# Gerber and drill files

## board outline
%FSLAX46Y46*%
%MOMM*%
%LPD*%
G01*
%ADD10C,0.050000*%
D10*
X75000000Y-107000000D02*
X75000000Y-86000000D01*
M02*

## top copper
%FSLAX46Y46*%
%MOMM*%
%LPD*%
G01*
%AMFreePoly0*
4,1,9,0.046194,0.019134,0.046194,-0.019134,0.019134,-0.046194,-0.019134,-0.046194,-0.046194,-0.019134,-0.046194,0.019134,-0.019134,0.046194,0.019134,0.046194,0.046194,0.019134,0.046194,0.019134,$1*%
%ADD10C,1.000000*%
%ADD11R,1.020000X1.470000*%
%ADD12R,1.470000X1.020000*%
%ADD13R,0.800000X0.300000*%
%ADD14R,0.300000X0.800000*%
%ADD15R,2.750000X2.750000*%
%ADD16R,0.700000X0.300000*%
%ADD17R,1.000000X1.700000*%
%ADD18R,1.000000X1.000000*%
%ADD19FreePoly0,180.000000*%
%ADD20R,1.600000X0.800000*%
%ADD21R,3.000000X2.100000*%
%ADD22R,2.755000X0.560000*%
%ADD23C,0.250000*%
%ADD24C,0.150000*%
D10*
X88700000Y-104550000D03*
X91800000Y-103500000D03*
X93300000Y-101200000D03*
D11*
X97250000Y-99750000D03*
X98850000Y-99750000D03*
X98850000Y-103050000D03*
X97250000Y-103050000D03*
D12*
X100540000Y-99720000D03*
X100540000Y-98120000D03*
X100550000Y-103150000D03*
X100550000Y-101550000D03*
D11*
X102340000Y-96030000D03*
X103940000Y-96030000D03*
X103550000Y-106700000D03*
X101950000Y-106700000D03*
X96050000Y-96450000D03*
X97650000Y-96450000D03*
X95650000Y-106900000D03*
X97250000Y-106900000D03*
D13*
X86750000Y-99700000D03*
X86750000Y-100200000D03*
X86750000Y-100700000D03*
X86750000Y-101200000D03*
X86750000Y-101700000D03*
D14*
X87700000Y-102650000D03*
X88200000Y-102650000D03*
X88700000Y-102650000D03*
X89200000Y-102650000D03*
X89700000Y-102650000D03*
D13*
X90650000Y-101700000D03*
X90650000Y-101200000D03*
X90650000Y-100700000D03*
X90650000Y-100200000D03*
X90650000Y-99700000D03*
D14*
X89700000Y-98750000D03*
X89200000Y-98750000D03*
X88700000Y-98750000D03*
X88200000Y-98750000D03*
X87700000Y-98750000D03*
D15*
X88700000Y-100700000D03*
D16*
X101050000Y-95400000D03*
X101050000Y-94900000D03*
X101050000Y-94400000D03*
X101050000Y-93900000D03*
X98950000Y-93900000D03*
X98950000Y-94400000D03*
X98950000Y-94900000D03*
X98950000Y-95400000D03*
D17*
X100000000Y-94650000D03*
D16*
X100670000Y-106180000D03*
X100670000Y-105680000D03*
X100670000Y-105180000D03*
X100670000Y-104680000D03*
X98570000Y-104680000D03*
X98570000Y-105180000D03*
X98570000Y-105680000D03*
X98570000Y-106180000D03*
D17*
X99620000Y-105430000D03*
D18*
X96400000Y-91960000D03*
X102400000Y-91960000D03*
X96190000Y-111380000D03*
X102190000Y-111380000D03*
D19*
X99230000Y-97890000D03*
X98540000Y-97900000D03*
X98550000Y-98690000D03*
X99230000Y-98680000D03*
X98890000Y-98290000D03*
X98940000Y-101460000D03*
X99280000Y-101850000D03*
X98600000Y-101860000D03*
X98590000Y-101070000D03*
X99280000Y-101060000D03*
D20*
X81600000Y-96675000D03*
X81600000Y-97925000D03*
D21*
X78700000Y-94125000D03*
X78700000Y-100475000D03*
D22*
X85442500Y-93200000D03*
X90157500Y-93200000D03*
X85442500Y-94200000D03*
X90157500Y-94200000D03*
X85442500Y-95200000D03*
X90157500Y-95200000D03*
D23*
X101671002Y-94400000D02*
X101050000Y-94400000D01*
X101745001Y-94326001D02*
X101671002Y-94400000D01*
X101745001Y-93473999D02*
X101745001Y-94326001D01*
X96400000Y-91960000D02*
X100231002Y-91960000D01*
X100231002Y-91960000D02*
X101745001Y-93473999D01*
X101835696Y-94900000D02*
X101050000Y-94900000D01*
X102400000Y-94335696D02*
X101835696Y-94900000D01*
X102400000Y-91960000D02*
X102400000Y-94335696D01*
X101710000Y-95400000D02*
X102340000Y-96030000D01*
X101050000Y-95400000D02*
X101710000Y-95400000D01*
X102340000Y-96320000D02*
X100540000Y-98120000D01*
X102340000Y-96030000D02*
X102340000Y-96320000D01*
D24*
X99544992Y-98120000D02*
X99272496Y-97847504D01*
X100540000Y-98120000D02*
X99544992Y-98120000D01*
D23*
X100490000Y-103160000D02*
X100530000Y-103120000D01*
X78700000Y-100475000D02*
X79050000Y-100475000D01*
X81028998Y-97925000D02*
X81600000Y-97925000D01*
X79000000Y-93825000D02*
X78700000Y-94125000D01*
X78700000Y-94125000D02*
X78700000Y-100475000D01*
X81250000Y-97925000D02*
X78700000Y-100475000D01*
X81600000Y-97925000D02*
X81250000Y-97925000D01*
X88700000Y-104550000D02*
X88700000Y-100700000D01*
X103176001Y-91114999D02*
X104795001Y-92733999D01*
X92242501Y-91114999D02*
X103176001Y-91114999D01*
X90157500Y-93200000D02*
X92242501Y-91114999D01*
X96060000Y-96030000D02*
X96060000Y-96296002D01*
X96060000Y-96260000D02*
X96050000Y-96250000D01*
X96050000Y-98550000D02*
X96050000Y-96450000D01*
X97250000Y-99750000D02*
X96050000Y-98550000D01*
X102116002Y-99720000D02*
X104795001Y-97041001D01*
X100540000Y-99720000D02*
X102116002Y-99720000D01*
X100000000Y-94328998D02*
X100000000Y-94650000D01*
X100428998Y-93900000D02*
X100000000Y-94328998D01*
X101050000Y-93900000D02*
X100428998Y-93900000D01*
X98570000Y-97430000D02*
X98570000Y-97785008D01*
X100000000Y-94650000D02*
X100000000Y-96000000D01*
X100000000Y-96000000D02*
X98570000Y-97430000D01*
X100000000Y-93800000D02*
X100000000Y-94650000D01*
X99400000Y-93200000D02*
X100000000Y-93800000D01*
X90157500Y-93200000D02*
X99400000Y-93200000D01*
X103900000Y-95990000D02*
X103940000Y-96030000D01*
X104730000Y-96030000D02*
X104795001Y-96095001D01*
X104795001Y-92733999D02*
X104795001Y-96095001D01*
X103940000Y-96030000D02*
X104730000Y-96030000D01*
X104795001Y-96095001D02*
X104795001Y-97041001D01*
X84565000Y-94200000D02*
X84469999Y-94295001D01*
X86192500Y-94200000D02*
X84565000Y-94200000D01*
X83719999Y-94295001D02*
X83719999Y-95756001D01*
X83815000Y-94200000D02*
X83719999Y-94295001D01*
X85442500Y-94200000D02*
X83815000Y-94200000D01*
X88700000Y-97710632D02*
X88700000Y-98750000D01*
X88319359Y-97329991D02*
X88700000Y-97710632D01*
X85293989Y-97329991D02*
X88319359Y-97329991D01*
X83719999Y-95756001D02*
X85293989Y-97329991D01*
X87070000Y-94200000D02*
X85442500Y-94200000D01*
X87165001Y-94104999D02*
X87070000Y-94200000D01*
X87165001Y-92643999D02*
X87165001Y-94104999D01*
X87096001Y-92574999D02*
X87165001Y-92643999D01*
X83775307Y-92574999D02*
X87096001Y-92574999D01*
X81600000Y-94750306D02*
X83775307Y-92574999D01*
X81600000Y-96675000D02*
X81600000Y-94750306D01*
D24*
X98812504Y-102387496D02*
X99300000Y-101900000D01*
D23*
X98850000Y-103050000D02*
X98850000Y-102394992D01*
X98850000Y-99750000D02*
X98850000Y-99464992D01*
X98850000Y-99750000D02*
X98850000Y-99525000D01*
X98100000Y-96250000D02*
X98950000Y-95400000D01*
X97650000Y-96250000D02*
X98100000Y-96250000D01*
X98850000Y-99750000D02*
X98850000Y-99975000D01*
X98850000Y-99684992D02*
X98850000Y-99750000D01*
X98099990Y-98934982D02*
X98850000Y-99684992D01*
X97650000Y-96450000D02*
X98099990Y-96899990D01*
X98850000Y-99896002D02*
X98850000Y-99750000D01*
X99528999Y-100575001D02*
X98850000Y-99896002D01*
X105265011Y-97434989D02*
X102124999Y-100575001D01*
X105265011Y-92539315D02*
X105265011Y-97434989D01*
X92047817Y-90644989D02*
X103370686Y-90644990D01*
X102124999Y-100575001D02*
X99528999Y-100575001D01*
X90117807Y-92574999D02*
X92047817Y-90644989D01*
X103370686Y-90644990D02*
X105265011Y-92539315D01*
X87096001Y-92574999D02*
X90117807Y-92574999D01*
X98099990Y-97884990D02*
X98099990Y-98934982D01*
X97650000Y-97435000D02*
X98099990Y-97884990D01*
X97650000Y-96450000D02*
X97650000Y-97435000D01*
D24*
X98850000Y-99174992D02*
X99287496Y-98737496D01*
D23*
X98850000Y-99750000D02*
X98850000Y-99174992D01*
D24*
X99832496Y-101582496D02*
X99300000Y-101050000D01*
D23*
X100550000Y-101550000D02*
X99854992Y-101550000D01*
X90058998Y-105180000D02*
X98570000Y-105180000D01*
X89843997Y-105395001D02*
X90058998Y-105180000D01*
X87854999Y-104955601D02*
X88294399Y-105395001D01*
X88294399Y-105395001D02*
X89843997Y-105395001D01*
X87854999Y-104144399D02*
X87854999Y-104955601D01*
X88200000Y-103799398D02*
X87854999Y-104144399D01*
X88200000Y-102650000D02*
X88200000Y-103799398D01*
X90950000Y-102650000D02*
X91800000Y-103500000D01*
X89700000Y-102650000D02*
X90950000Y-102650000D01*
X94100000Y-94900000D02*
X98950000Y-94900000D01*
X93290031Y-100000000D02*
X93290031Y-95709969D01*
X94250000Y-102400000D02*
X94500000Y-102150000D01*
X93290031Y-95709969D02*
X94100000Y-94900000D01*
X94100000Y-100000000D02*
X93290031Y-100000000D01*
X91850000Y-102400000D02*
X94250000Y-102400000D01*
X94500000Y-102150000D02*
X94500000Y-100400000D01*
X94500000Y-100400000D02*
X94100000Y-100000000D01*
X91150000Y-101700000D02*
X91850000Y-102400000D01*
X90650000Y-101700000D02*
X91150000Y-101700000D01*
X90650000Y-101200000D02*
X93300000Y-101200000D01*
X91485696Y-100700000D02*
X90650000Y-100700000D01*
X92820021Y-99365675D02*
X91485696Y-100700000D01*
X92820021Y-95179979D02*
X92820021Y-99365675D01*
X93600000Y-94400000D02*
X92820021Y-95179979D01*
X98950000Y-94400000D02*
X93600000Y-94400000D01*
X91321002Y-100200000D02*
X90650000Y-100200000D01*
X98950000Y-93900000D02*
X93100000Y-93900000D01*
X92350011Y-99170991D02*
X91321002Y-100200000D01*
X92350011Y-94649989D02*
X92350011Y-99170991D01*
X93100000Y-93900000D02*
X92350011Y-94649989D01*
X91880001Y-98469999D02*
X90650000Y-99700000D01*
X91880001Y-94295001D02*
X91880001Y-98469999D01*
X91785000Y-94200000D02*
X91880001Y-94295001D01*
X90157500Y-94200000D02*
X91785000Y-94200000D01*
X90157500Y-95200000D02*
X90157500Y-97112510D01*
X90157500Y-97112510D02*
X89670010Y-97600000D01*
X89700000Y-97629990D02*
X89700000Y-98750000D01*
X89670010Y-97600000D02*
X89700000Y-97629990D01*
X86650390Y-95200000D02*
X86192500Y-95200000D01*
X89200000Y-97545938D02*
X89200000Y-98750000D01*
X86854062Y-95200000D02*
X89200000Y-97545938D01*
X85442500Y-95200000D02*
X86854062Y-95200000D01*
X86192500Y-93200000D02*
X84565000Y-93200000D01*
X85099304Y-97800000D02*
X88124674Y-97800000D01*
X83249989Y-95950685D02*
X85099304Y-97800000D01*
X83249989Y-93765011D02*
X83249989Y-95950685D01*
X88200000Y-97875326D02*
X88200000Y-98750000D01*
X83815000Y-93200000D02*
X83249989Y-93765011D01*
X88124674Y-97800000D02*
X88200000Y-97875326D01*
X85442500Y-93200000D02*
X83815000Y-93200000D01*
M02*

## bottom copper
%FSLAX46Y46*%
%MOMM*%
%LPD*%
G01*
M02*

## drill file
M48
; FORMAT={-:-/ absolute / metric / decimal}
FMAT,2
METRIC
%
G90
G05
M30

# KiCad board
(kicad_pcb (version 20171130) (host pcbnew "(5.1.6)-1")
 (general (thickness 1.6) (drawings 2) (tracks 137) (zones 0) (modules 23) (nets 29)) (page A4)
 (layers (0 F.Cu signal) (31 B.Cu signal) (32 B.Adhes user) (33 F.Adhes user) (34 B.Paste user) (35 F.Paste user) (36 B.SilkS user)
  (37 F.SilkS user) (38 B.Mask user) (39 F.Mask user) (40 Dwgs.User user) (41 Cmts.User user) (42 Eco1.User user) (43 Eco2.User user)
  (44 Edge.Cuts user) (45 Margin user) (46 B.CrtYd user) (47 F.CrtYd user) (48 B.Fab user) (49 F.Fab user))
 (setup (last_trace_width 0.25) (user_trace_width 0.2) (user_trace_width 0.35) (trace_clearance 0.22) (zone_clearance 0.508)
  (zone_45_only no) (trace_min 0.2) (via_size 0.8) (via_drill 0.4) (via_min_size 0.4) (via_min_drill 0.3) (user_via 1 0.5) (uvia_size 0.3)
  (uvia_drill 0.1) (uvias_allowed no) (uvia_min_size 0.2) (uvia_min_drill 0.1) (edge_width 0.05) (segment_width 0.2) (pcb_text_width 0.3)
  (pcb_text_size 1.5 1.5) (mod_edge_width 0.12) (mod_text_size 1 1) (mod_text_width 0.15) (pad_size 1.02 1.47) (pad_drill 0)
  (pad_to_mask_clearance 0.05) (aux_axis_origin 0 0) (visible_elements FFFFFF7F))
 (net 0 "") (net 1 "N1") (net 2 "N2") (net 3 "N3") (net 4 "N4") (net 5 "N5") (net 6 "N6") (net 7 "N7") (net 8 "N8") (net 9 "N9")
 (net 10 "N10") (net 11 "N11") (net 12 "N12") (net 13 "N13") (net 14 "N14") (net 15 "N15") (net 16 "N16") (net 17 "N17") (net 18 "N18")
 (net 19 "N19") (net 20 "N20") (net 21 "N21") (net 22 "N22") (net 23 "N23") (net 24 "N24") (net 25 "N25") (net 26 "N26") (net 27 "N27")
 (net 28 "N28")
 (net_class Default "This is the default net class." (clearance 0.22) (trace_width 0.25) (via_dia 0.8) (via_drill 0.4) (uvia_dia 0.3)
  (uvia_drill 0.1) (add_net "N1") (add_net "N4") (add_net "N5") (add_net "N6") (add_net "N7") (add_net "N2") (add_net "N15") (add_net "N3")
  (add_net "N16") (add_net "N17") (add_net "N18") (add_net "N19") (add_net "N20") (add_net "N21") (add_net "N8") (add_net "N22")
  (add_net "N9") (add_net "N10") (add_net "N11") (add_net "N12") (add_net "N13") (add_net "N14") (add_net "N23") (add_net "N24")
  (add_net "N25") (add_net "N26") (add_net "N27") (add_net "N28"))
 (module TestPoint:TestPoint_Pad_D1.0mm (layer F.Cu) (at 88.7 104.55)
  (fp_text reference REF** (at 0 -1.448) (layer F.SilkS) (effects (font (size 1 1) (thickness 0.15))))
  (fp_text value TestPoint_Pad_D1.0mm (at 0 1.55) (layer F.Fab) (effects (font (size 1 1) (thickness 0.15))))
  (pad 1 smd circle (at 0 0) (size 1 1) (layers F.Cu F.Mask) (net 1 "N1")))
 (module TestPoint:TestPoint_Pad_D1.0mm (layer F.Cu) (at 91.8 103.5)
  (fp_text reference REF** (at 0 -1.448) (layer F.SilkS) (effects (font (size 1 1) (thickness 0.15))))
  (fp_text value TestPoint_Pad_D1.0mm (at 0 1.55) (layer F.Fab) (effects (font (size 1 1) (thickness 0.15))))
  (pad 1 smd circle (at 0 0) (size 1 1) (layers F.Cu F.Mask) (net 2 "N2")))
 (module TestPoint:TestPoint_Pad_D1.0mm (layer F.Cu) (at 93.3 101.2)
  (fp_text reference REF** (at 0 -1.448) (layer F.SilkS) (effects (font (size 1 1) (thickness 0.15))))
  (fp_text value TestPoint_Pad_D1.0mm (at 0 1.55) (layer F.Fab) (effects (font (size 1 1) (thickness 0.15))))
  (pad 1 smd circle (at 0 0) (size 1 1) (layers F.Cu F.Mask) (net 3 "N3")))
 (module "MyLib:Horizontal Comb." (layer F.Cu) (at 119.7 96.4)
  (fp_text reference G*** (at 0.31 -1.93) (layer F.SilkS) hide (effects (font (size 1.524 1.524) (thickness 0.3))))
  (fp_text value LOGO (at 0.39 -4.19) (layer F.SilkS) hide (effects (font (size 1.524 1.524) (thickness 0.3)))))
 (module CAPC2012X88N (layer F.Cu) (at 98.05 99.75)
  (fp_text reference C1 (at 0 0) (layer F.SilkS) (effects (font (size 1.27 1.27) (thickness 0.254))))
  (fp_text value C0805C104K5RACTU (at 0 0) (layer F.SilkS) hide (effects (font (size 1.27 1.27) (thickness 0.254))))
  (pad 1 smd rect (at -0.8 0) (size 1.02 1.47) (layers F.Cu F.Paste F.Mask) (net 1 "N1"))
  (pad 2 smd rect (at 0.8 0) (size 1.02 1.47) (layers F.Cu F.Paste F.Mask) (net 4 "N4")))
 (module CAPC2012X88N (layer F.Cu) (at 98.05 103.05)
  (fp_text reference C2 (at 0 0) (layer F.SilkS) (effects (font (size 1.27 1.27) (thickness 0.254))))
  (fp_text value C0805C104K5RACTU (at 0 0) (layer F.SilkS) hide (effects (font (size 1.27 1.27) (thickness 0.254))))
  (pad 2 smd rect (at 0.8 0) (size 1.02 1.47) (layers F.Cu F.Paste F.Mask) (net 4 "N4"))
  (pad 1 smd rect (at -0.8 0) (size 1.02 1.47) (layers F.Cu F.Paste F.Mask) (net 1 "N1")))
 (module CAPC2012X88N (layer F.Cu) (at 100.54 98.92 90)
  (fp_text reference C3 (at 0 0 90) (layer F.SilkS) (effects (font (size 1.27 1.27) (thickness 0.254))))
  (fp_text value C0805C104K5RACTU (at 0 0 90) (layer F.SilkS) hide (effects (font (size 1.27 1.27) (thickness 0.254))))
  (pad 1 smd rect (at -0.8 0 90) (size 1.02 1.47) (layers F.Cu F.Paste F.Mask) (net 1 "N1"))
  (pad 2 smd rect (at 0.8 0 90) (size 1.02 1.47) (layers F.Cu F.Paste F.Mask) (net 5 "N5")))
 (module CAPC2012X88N (layer F.Cu) (at 100.55 102.35 90)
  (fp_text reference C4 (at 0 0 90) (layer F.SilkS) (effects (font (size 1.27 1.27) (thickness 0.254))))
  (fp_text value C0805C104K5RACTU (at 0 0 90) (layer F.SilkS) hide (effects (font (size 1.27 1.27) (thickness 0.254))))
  (pad 1 smd rect (at -0.8 0 90) (size 1.02 1.47) (layers F.Cu F.Paste F.Mask) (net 1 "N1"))
  (pad 2 smd rect (at 0.8 0 90) (size 1.02 1.47) (layers F.Cu F.Paste F.Mask) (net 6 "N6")))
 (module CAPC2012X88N (layer F.Cu) (at 103.14 96.03 180)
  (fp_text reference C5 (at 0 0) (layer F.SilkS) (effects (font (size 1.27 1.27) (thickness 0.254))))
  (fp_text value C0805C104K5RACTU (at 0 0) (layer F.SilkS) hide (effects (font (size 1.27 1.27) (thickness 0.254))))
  (pad 2 smd rect (at 0.8 0 180) (size 1.02 1.47) (layers F.Cu F.Paste F.Mask) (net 5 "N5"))
  (pad 1 smd rect (at -0.8 0 180) (size 1.02 1.47) (layers F.Cu F.Paste F.Mask) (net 1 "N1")))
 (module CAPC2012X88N (layer F.Cu) (at 102.75 106.7 180)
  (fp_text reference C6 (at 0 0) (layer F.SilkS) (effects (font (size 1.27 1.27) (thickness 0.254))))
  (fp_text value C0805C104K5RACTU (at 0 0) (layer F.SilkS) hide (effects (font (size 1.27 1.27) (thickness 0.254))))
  (pad 1 smd rect (at -0.8 0 180) (size 1.02 1.47) (layers F.Cu F.Paste F.Mask) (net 1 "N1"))
  (pad 2 smd rect (at 0.8 0 180) (size 1.02 1.47) (layers F.Cu F.Paste F.Mask) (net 6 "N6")))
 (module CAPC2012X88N (layer F.Cu) (at 96.85 96.45)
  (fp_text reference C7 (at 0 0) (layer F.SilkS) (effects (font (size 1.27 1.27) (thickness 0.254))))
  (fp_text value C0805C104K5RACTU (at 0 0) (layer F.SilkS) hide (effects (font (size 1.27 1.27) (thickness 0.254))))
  (pad 1 smd rect (at -0.8 0) (size 1.02 1.47) (layers F.Cu F.Paste F.Mask) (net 1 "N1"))
  (pad 2 smd rect (at 0.8 0) (size 1.02 1.47) (layers F.Cu F.Paste F.Mask) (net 4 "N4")))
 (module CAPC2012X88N (layer F.Cu) (at 96.45 106.9)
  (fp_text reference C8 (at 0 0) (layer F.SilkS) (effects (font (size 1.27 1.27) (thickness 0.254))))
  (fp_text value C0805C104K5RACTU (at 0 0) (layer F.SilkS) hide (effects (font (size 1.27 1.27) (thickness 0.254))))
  (pad 1 smd rect (at -0.8 0) (size 1.02 1.47) (layers F.Cu F.Paste F.Mask) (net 1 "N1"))
  (pad 2 smd rect (at 0.8 0) (size 1.02 1.47) (layers F.Cu F.Paste F.Mask) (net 4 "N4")))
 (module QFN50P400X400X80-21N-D (layer F.Cu) (at 88.7 100.7)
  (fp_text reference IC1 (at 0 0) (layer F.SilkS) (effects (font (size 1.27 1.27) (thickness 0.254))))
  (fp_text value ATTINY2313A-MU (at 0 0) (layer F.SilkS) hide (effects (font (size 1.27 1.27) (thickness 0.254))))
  (pad 1 smd rect (at -1.95 -1 90) (size 0.3 0.8) (layers F.Cu F.Paste F.Mask) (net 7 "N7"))
  (pad 2 smd rect (at -1.95 -0.5 90) (size 0.3 0.8) (layers F.Cu F.Paste F.Mask) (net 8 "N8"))
  (pad 3 smd rect (at -1.95 0 90) (size 0.3 0.8) (layers F.Cu F.Paste F.Mask) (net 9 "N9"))
  (pad 4 smd rect (at -1.95 0.5 90) (size 0.3 0.8) (layers F.Cu F.Paste F.Mask) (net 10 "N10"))
  (pad 5 smd rect (at -1.95 1 90) (size 0.3 0.8) (layers F.Cu F.Paste F.Mask) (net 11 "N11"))
  (pad 6 smd rect (at -1 1.95) (size 0.3 0.8) (layers F.Cu F.Paste F.Mask) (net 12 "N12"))
  (pad 7 smd rect (at -0.5 1.95) (size 0.3 0.8) (layers F.Cu F.Paste F.Mask) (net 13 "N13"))
  (pad 8 smd rect (at 0 1.95) (size 0.3 0.8) (layers F.Cu F.Paste F.Mask) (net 1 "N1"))
  (pad 9 smd rect (at 0.5 1.95) (size 0.3 0.8) (layers F.Cu F.Paste F.Mask) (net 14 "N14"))
  (pad 10 smd rect (at 1 1.95) (size 0.3 0.8) (layers F.Cu F.Paste F.Mask) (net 2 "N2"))
  (pad 11 smd rect (at 1.95 1 90) (size 0.3 0.8) (layers F.Cu F.Paste F.Mask) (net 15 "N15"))
  (pad 12 smd rect (at 1.95 0.5 90) (size 0.3 0.8) (layers F.Cu F.Paste F.Mask) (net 3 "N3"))
  (pad 13 smd rect (at 1.95 0 90) (size 0.3 0.8) (layers F.Cu F.Paste F.Mask) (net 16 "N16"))
  (pad 14 smd rect (at 1.95 -0.5 90) (size 0.3 0.8) (layers F.Cu F.Paste F.Mask) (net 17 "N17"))
  (pad 15 smd rect (at 1.95 -1 90) (size 0.3 0.8) (layers F.Cu F.Paste F.Mask) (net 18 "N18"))
  (pad 16 smd rect (at 1 -1.95) (size 0.3 0.8) (layers F.Cu F.Paste F.Mask) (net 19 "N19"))
  (pad 17 smd rect (at 0.5 -1.95) (size 0.3 0.8) (layers F.Cu F.Paste F.Mask) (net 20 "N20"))
  (pad 18 smd rect (at 0 -1.95) (size 0.3 0.8) (layers F.Cu F.Paste F.Mask) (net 4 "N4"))
  (pad 19 smd rect (at -0.5 -1.95) (size 0.3 0.8) (layers F.Cu F.Paste F.Mask) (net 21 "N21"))
  (pad 20 smd rect (at -1 -1.95) (size 0.3 0.8) (layers F.Cu F.Paste F.Mask) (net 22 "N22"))
  (pad 21 smd rect (at 0 0) (size 2.75 2.75) (layers F.Cu F.Paste F.Mask) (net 1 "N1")))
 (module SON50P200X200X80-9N (layer F.Cu) (at 100 94.65 180)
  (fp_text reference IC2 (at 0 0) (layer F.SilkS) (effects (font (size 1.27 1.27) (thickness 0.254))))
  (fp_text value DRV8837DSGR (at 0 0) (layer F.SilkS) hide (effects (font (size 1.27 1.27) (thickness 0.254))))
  (pad 1 smd rect (at -1.05 -0.75 270) (size 0.3 0.7) (layers F.Cu F.Paste F.Mask) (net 5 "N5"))
  (pad 2 smd rect (at -1.05 -0.25 270) (size 0.3 0.7) (layers F.Cu F.Paste F.Mask) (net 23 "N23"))
  (pad 3 smd rect (at -1.05 0.25 270) (size 0.3 0.7) (layers F.Cu F.Paste F.Mask) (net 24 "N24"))
  (pad 4 smd rect (at -1.05 0.75 270) (size 0.3 0.7) (layers F.Cu F.Paste F.Mask) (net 1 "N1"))
  (pad 5 smd rect (at 1.05 0.75 270) (size 0.3 0.7) (layers F.Cu F.Paste F.Mask) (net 17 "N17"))
  (pad 6 smd rect (at 1.05 0.25 270) (size 0.3 0.7) (layers F.Cu F.Paste F.Mask) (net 16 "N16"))
  (pad 7 smd rect (at 1.05 -0.25 270) (size 0.3 0.7) (layers F.Cu F.Paste F.Mask) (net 15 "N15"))
  (pad 8 smd rect (at 1.05 -0.75 270) (size 0.3 0.7) (layers F.Cu F.Paste F.Mask) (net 4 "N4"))
  (pad 9 smd rect (at 0 0 180) (size 1 1.7) (layers F.Cu F.Paste F.Mask) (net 1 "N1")))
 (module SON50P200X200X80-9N (layer F.Cu) (at 99.62 105.43 180)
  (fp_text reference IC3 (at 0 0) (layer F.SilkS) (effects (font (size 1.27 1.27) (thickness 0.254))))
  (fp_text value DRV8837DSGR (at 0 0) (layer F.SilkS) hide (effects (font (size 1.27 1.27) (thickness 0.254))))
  (pad 1 smd rect (at -1.05 -0.75 270) (size 0.3 0.7) (layers F.Cu F.Paste F.Mask) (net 6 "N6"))
  (pad 2 smd rect (at -1.05 -0.25 270) (size 0.3 0.7) (layers F.Cu F.Paste F.Mask) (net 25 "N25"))
  (pad 3 smd rect (at -1.05 0.25 270) (size 0.3 0.7) (layers F.Cu F.Paste F.Mask) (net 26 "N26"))
  (pad 4 smd rect (at -1.05 0.75 270) (size 0.3 0.7) (layers F.Cu F.Paste F.Mask) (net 1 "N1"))
  (pad 5 smd rect (at 1.05 0.75 270) (size 0.3 0.7) (layers F.Cu F.Paste F.Mask) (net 3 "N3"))
  (pad 6 smd rect (at 1.05 0.25 270) (size 0.3 0.7) (layers F.Cu F.Paste F.Mask) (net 13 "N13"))
  (pad 7 smd rect (at 1.05 -0.25 270) (size 0.3 0.7) (layers F.Cu F.Paste F.Mask) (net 2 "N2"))
  (pad 8 smd rect (at 1.05 -0.75 270) (size 0.3 0.7) (layers F.Cu F.Paste F.Mask) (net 4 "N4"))
  (pad 9 smd rect (at 0 0 180) (size 1 1.7) (layers F.Cu F.Paste F.Mask) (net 1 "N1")))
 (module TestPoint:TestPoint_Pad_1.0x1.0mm (layer F.Cu) (at 96.4 91.96)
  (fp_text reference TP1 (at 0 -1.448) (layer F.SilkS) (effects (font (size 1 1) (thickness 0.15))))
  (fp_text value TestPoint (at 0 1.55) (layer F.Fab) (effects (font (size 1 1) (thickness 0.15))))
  (pad 1 smd rect (at 0 0) (size 1 1) (layers F.Cu F.Mask) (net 24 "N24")))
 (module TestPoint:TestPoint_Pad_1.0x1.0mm (layer F.Cu) (at 102.4 91.96)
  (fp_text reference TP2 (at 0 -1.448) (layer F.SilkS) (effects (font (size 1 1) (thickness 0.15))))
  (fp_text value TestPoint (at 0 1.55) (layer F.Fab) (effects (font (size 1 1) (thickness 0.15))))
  (pad 1 smd rect (at 0 0) (size 1 1) (layers F.Cu F.Mask) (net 23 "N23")))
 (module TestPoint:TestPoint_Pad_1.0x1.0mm (layer F.Cu) (at 96.19 111.38)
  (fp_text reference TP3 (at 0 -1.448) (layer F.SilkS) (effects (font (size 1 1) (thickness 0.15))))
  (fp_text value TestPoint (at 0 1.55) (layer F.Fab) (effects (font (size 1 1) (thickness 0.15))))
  (pad 1 smd rect (at 0 0) (size 1 1) (layers F.Cu F.Mask) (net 25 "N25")))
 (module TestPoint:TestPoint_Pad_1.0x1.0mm (layer F.Cu) (at 102.19 111.38)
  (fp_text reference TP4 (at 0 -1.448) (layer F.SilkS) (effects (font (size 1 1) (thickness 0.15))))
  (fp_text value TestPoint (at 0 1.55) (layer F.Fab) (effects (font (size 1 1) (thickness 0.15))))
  (pad 1 smd rect (at 0 0) (size 1 1) (layers F.Cu F.Mask) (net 26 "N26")))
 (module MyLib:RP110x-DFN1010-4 (layer F.Cu) (at 99.45 97.73 180)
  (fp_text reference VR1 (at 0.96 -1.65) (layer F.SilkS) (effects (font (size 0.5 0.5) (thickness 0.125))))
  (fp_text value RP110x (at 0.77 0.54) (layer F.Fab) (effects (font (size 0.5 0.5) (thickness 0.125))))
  (pad 1 smd custom (at 0.22 -0.16 180) (size 0.1 0.1) (layers F.Cu F.Paste F.Mask) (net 5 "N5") (zone_connect 0)
   (options (clearance outline) (anchor circle)) (primitives))
  (pad 2 smd custom (at 0.91 -0.17 180) (size 0.1 0.1) (layers F.Cu F.Paste F.Mask) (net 1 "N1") (zone_connect 0)
   (options (clearance outline) (anchor circle)) (primitives))
  (pad 3 smd custom (at 0.9 -0.96 180) (size 0.1 0.1) (layers F.Cu F.Paste F.Mask) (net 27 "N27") (zone_connect 0)
   (options (clearance outline) (anchor circle)) (primitives))
  (pad 4 smd custom (at 0.22 -0.95 180) (size 0.1 0.1) (layers F.Cu F.Paste F.Mask) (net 4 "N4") (zone_connect 0)
   (options (clearance outline) (anchor circle)) (primitives))
  (pad 5 smd custom (at 0.56 -0.56 180) (size 0.1 0.1) (layers F.Cu F.Paste F.Mask) (zone_connect 0)
   (options (clearance outline) (anchor circle)) (primitives)))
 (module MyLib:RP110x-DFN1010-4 (layer F.Cu) (at 99.5 100.9 180)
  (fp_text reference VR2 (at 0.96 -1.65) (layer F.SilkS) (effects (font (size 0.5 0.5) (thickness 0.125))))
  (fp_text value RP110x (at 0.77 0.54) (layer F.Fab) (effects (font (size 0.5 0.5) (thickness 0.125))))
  (pad 5 smd custom (at 0.56 -0.56 180) (size 0.1 0.1) (layers F.Cu F.Paste F.Mask) (zone_connect 0)
   (options (clearance outline) (anchor circle)) (primitives))
  (pad 4 smd custom (at 0.22 -0.95 180) (size 0.1 0.1) (layers F.Cu F.Paste F.Mask) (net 4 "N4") (zone_connect 0)
   (options (clearance outline) (anchor circle)) (primitives))
  (pad 3 smd custom (at 0.9 -0.96 180) (size 0.1 0.1) (layers F.Cu F.Paste F.Mask) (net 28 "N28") (zone_connect 0)
   (options (clearance outline) (anchor circle)) (primitives))
  (pad 2 smd custom (at 0.91 -0.17 180) (size 0.1 0.1) (layers F.Cu F.Paste F.Mask) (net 1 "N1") (zone_connect 0)
   (options (clearance outline) (anchor circle)) (primitives))
  (pad 1 smd custom (at 0.22 -0.16 180) (size 0.1 0.1) (layers F.Cu F.Paste F.Mask) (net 6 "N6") (zone_connect 0)
   (options (clearance outline) (anchor circle)) (primitives)))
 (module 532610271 (layer F.Cu) (at 79.3 97.3 90)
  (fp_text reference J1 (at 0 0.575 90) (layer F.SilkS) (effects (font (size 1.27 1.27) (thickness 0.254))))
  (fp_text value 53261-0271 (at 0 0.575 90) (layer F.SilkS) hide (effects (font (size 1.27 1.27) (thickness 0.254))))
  (pad 1 smd rect (at 0.625 2.3 90) (size 0.8 1.6) (layers F.Cu F.Paste F.Mask) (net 4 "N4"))
  (pad 2 smd rect (at -0.625 2.3 90) (size 0.8 1.6) (layers F.Cu F.Paste F.Mask) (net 1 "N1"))
  (pad MP1 smd rect (at 3.175 -0.6 90) (size 2.1 3) (layers F.Cu F.Paste F.Mask) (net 1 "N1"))
  (pad MP2 smd rect (at -3.175 -0.6 90) (size 2.1 3) (layers F.Cu F.Paste F.Mask) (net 1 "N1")))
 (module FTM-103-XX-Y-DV (layer F.Cu) (at 87.8 94.2 270)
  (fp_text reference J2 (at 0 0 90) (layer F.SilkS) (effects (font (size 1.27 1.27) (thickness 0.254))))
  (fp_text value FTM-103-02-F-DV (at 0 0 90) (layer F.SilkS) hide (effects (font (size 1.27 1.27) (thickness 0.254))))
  (pad 1 smd rect (at -1 2.3575 270) (size 0.56 2.755) (layers F.Cu F.Paste F.Mask) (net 21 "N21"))
  (pad 2 smd rect (at -1 -2.3575 270) (size 0.56 2.755) (layers F.Cu F.Paste F.Mask) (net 1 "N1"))
  (pad 3 smd rect (at 0 2.3575 270) (size 0.56 2.755) (layers F.Cu F.Paste F.Mask) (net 4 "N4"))
  (pad 4 smd rect (at 0 -2.3575 270) (size 0.56 2.755) (layers F.Cu F.Paste F.Mask) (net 18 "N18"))
  (pad 5 smd rect (at 1 2.3575 270) (size 0.56 2.755) (layers F.Cu F.Paste F.Mask) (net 20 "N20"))
  (pad 6 smd rect (at 1 -2.3575 270) (size 0.56 2.755) (layers F.Cu F.Paste F.Mask) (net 19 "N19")))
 (gr_line (start 75 107) (end 75 86) (layer Edge.Cuts) (width 0.05))
 (segment (start 101.671002 94.4) (end 101.05 94.4) (width 0.25) (layer F.Cu) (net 24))
 (segment (start 101.745001 94.326001) (end 101.671002 94.4) (width 0.25) (layer F.Cu) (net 24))
 (segment (start 101.745001 93.473999) (end 101.745001 94.326001) (width 0.25) (layer F.Cu) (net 24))
 (segment (start 96.4 91.96) (end 100.231002 91.96) (width 0.25) (layer F.Cu) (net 24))
 (segment (start 100.231002 91.96) (end 101.745001 93.473999) (width 0.25) (layer F.Cu) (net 24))
 (segment (start 101.835696 94.9) (end 101.05 94.9) (width 0.25) (layer F.Cu) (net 23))
 (segment (start 102.4 94.335696) (end 101.835696 94.9) (width 0.25) (layer F.Cu) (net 23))
 (segment (start 102.4 91.96) (end 102.4 94.335696) (width 0.25) (layer F.Cu) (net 23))
 (segment (start 101.71 95.4) (end 102.34 96.03) (width 0.25) (layer F.Cu) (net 5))
 (segment (start 101.05 95.4) (end 101.71 95.4) (width 0.25) (layer F.Cu) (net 5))
 (segment (start 102.34 96.32) (end 100.54 98.12) (width 0.25) (layer F.Cu) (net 5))
 (segment (start 102.34 96.03) (end 102.34 96.32) (width 0.25) (layer F.Cu) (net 5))
 (segment (start 99.544992 98.12) (end 99.272496 97.847504) (width 0.15) (layer F.Cu) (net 5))
 (segment (start 100.54 98.12) (end 99.544992 98.12) (width 0.15) (layer F.Cu) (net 5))
 (segment (start 100.49 103.16) (end 100.53 103.12) (width 0.25) (layer F.Cu) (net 1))
 (segment (start 78.7 100.475) (end 79.05 100.475) (width 0.25) (layer F.Cu) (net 1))
 (segment (start 81.028998 97.925) (end 81.6 97.925) (width 0.25) (layer F.Cu) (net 1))
 (segment (start 79 93.825) (end 78.7 94.125) (width 0.25) (layer F.Cu) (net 1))
 (segment (start 78.7 94.125) (end 78.7 100.475) (width 0.25) (layer F.Cu) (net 1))
 (segment (start 81.25 97.925) (end 78.7 100.475) (width 0.25) (layer F.Cu) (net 1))
 (segment (start 81.6 97.925) (end 81.25 97.925) (width 0.25) (layer F.Cu) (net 1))
 (segment (start 88.7 104.55) (end 88.7 100.7) (width 0.25) (layer F.Cu) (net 1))
 (segment (start 103.176001 91.114999) (end 104.795001 92.733999) (width 0.25) (layer F.Cu) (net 1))
 (segment (start 92.242501 91.114999) (end 103.176001 91.114999) (width 0.25) (layer F.Cu) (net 1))
 (segment (start 90.1575 93.2) (end 92.242501 91.114999) (width 0.25) (layer F.Cu) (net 1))
 (segment (start 96.06 96.03) (end 96.06 96.296002) (width 0.25) (layer F.Cu) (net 1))
 (segment (start 96.06 96.26) (end 96.05 96.25) (width 0.25) (layer F.Cu) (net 1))
 (segment (start 96.05 98.55) (end 96.05 96.45) (width 0.25) (layer F.Cu) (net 1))
 (segment (start 97.25 99.75) (end 96.05 98.55) (width 0.25) (layer F.Cu) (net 1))
 (segment (start 102.116002 99.72) (end 104.795001 97.041001) (width 0.25) (layer F.Cu) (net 1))
 (segment (start 100.54 99.72) (end 102.116002 99.72) (width 0.25) (layer F.Cu) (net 1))
 (segment (start 100 94.328998) (end 100 94.65) (width 0.25) (layer F.Cu) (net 1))
 (segment (start 100.428998 93.9) (end 100 94.328998) (width 0.25) (layer F.Cu) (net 1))
 (segment (start 101.05 93.9) (end 100.428998 93.9) (width 0.25) (layer F.Cu) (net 1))
 (segment (start 98.57 97.43) (end 98.57 97.785008) (width 0.25) (layer F.Cu) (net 1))
 (segment (start 100 94.65) (end 100 96) (width 0.25) (layer F.Cu) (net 1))
 (segment (start 100 96) (end 98.57 97.43) (width 0.25) (layer F.Cu) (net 1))
 (segment (start 100 93.8) (end 100 94.65) (width 0.25) (layer F.Cu) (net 1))
 (segment (start 99.4 93.2) (end 100 93.8) (width 0.25) (layer F.Cu) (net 1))
 (segment (start 90.1575 93.2) (end 99.4 93.2) (width 0.25) (layer F.Cu) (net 1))
 (segment (start 103.9 95.99) (end 103.94 96.03) (width 0.25) (layer F.Cu) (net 1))
 (segment (start 104.73 96.03) (end 104.795001 96.095001) (width 0.25) (layer F.Cu) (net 1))
 (segment (start 104.795001 92.733999) (end 104.795001 96.095001) (width 0.25) (layer F.Cu) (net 1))
 (segment (start 103.94 96.03) (end 104.73 96.03) (width 0.25) (layer F.Cu) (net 1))
 (segment (start 104.795001 96.095001) (end 104.795001 97.041001) (width 0.25) (layer F.Cu) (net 1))
 (segment (start 84.565 94.2) (end 84.469999 94.295001) (width 0.25) (layer F.Cu) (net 4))
 (segment (start 86.1925 94.2) (end 84.565 94.2) (width 0.25) (layer F.Cu) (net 4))
 (segment (start 83.719999 94.295001) (end 83.719999 95.756001) (width 0.25) (layer F.Cu) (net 4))
 (segment (start 83.815 94.2) (end 83.719999 94.295001) (width 0.25) (layer F.Cu) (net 4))
 (segment (start 85.4425 94.2) (end 83.815 94.2) (width 0.25) (layer F.Cu) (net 4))
 (segment (start 88.7 97.710632) (end 88.7 98.75) (width 0.25) (layer F.Cu) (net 4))
 (segment (start 88.319359 97.329991) (end 88.7 97.710632) (width 0.25) (layer F.Cu) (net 4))
 (segment (start 85.293989 97.329991) (end 88.319359 97.329991) (width 0.25) (layer F.Cu) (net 4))
 (segment (start 83.719999 95.756001) (end 85.293989 97.329991) (width 0.25) (layer F.Cu) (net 4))
 (segment (start 87.07 94.2) (end 85.4425 94.2) (width 0.25) (layer F.Cu) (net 4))
 (segment (start 87.165001 94.104999) (end 87.07 94.2) (width 0.25) (layer F.Cu) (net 4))
 (segment (start 87.165001 92.643999) (end 87.165001 94.104999) (width 0.25) (layer F.Cu) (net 4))
 (segment (start 87.096001 92.574999) (end 87.165001 92.643999) (width 0.25) (layer F.Cu) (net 4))
 (segment (start 83.775307 92.574999) (end 87.096001 92.574999) (width 0.25) (layer F.Cu) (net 4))
 (segment (start 81.6 94.750306) (end 83.775307 92.574999) (width 0.25) (layer F.Cu) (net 4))
 (segment (start 81.6 96.675) (end 81.6 94.750306) (width 0.25) (layer F.Cu) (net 4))
 (segment (start 98.812504 102.387496) (end 99.3 101.9) (width 0.15) (layer F.Cu) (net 4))
 (segment (start 98.85 103.05) (end 98.85 102.394992) (width 0.25) (layer F.Cu) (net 4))
 (segment (start 98.85 99.75) (end 98.85 99.464992) (width 0.25) (layer F.Cu) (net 4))
 (segment (start 98.85 99.75) (end 98.85 99.525) (width 0.25) (layer F.Cu) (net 4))
 (segment (start 98.1 96.25) (end 98.95 95.4) (width 0.25) (layer F.Cu) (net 4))
 (segment (start 97.65 96.25) (end 98.1 96.25) (width 0.25) (layer F.Cu) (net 4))
 (segment (start 98.85 99.75) (end 98.85 99.975) (width 0.25) (layer F.Cu) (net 4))
 (segment (start 98.85 99.684992) (end 98.85 99.75) (width 0.25) (layer F.Cu) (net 4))
 (segment (start 98.09999 98.934982) (end 98.85 99.684992) (width 0.25) (layer F.Cu) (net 4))
 (segment (start 97.65 96.45) (end 98.09999 96.89999) (width 0.25) (layer F.Cu) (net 4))
 (segment (start 98.85 99.896002) (end 98.85 99.75) (width 0.25) (layer F.Cu) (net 4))
 (segment (start 99.528999 100.575001) (end 98.85 99.896002) (width 0.25) (layer F.Cu) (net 4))
 (segment (start 105.265011 97.434989) (end 102.124999 100.575001) (width 0.25) (layer F.Cu) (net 4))
 (segment (start 105.265011 92.539315) (end 105.265011 97.434989) (width 0.25) (layer F.Cu) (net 4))
 (segment (start 92.047817 90.644989) (end 103.370686 90.64499) (width 0.25) (layer F.Cu) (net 4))
 (segment (start 102.124999 100.575001) (end 99.528999 100.575001) (width 0.25) (layer F.Cu) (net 4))
 (segment (start 90.117807 92.574999) (end 92.047817 90.644989) (width 0.25) (layer F.Cu) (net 4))
 (segment (start 103.370686 90.64499) (end 105.265011 92.539315) (width 0.25) (layer F.Cu) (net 4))
 (segment (start 87.096001 92.574999) (end 90.117807 92.574999) (width 0.25) (layer F.Cu) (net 4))
 (segment (start 98.09999 97.88499) (end 98.09999 98.934982) (width 0.25) (layer F.Cu) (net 4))
 (segment (start 97.65 97.435) (end 98.09999 97.88499) (width 0.25) (layer F.Cu) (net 4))
 (segment (start 97.65 96.45) (end 97.65 97.435) (width 0.25) (layer F.Cu) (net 4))
 (segment (start 98.85 99.174992) (end 99.287496 98.737496) (width 0.15) (layer F.Cu) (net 4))
 (segment (start 98.85 99.75) (end 98.85 99.174992) (width 0.25) (layer F.Cu) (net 4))
 (segment (start 99.832496 101.582496) (end 99.3 101.05) (width 0.15) (layer F.Cu) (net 6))
 (segment (start 100.55 101.55) (end 99.854992 101.55) (width 0.25) (layer F.Cu) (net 6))
 (segment (start 90.058998 105.18) (end 98.57 105.18) (width 0.25) (layer F.Cu) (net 13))
 (segment (start 89.843997 105.395001) (end 90.058998 105.18) (width 0.25) (layer F.Cu) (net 13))
 (segment (start 87.854999 104.955601) (end 88.294399 105.395001) (width 0.25) (layer F.Cu) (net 13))
 (segment (start 88.294399 105.395001) (end 89.843997 105.395001) (width 0.25) (layer F.Cu) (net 13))
 (segment (start 87.854999 104.144399) (end 87.854999 104.955601) (width 0.25) (layer F.Cu) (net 13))
 (segment (start 88.2 103.799398) (end 87.854999 104.144399) (width 0.25) (layer F.Cu) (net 13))
 (segment (start 88.2 102.65) (end 88.2 103.799398) (width 0.25) (layer F.Cu) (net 13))
 (segment (start 90.95 102.65) (end 91.8 103.5) (width 0.25) (layer F.Cu) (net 2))
 (segment (start 89.7 102.65) (end 90.95 102.65) (width 0.25) (layer F.Cu) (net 2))
 (segment (start 94.1 94.9) (end 98.95 94.9) (width 0.25) (layer F.Cu) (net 15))
 (segment (start 93.290031 100) (end 93.290031 95.709969) (width 0.25) (layer F.Cu) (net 15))
 (segment (start 94.25 102.4) (end 94.5 102.15) (width 0.25) (layer F.Cu) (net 15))
 (segment (start 93.290031 95.709969) (end 94.1 94.9) (width 0.25) (layer F.Cu) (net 15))
 (segment (start 94.1 100) (end 93.290031 100) (width 0.25) (layer F.Cu) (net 15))
 (segment (start 91.85 102.4) (end 94.25 102.4) (width 0.25) (layer F.Cu) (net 15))
 (segment (start 94.5 102.15) (end 94.5 100.4) (width 0.25) (layer F.Cu) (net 15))
 (segment (start 94.5 100.4) (end 94.1 100) (width 0.25) (layer F.Cu) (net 15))
 (segment (start 91.15 101.7) (end 91.85 102.4) (width 0.25) (layer F.Cu) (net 15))
 (segment (start 90.65 101.7) (end 91.15 101.7) (width 0.25) (layer F.Cu) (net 15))
 (segment (start 90.65 101.2) (end 93.3 101.2) (width 0.25) (layer F.Cu) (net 3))
 (segment (start 91.485696 100.7) (end 90.65 100.7) (width 0.25) (layer F.Cu) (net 16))
 (segment (start 92.820021 99.365675) (end 91.485696 100.7) (width 0.25) (layer F.Cu) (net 16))
 (segment (start 92.820021 95.179979) (end 92.820021 99.365675) (width 0.25) (layer F.Cu) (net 16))
 (segment (start 93.6 94.4) (end 92.820021 95.179979) (width 0.25) (layer F.Cu) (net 16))
 (segment (start 98.95 94.4) (end 93.6 94.4) (width 0.25) (layer F.Cu) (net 16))
 (segment (start 91.321002 100.2) (end 90.65 100.2) (width 0.25) (layer F.Cu) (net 17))
 (segment (start 98.95 93.9) (end 93.1 93.9) (width 0.25) (layer F.Cu) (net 17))
 (segment (start 92.350011 99.170991) (end 91.321002 100.2) (width 0.25) (layer F.Cu) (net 17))
 (segment (start 92.350011 94.649989) (end 92.350011 99.170991) (width 0.25) (layer F.Cu) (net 17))
 (segment (start 93.1 93.9) (end 92.350011 94.649989) (width 0.25) (layer F.Cu) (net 17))
 (segment (start 91.880001 98.469999) (end 90.65 99.7) (width 0.25) (layer F.Cu) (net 18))
 (segment (start 91.880001 94.295001) (end 91.880001 98.469999) (width 0.25) (layer F.Cu) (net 18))
 (segment (start 91.785 94.2) (end 91.880001 94.295001) (width 0.25) (layer F.Cu) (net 18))
 (segment (start 90.1575 94.2) (end 91.785 94.2) (width 0.25) (layer F.Cu) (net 18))
 (segment (start 90.1575 95.2) (end 90.1575 97.11251) (width 0.25) (layer F.Cu) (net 19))
 (segment (start 90.1575 97.11251) (end 89.67001 97.6) (width 0.25) (layer F.Cu) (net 19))
 (segment (start 89.7 97.62999) (end 89.7 98.75) (width 0.25) (layer F.Cu) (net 19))
 (segment (start 89.67001 97.6) (end 89.7 97.62999) (width 0.25) (layer F.Cu) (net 19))
 (segment (start 86.65039 95.2) (end 86.1925 95.2) (width 0.25) (layer F.Cu) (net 20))
 (segment (start 89.2 97.545938) (end 89.2 98.75) (width 0.25) (layer F.Cu) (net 20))
 (segment (start 86.854062 95.2) (end 89.2 97.545938) (width 0.25) (layer F.Cu) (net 20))
 (segment (start 85.4425 95.2) (end 86.854062 95.2) (width 0.25) (layer F.Cu) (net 20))
 (segment (start 86.1925 93.2) (end 84.565 93.2) (width 0.25) (layer F.Cu) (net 21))
 (segment (start 85.099304 97.8) (end 88.124674 97.8) (width 0.25) (layer F.Cu) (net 21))
 (segment (start 83.249989 95.950685) (end 85.099304 97.8) (width 0.25) (layer F.Cu) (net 21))
 (segment (start 83.249989 93.765011) (end 83.249989 95.950685) (width 0.25) (layer F.Cu) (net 21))
 (segment (start 88.2 97.875326) (end 88.2 98.75) (width 0.25) (layer F.Cu) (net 21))
 (segment (start 83.815 93.2) (end 83.249989 93.765011) (width 0.25) (layer F.Cu) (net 21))
 (segment (start 88.124674 97.8) (end 88.2 97.875326) (width 0.25) (layer F.Cu) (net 21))
 (segment (start 85.4425 93.2) (end 83.815 93.2) (width 0.25) (layer F.Cu) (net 21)))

